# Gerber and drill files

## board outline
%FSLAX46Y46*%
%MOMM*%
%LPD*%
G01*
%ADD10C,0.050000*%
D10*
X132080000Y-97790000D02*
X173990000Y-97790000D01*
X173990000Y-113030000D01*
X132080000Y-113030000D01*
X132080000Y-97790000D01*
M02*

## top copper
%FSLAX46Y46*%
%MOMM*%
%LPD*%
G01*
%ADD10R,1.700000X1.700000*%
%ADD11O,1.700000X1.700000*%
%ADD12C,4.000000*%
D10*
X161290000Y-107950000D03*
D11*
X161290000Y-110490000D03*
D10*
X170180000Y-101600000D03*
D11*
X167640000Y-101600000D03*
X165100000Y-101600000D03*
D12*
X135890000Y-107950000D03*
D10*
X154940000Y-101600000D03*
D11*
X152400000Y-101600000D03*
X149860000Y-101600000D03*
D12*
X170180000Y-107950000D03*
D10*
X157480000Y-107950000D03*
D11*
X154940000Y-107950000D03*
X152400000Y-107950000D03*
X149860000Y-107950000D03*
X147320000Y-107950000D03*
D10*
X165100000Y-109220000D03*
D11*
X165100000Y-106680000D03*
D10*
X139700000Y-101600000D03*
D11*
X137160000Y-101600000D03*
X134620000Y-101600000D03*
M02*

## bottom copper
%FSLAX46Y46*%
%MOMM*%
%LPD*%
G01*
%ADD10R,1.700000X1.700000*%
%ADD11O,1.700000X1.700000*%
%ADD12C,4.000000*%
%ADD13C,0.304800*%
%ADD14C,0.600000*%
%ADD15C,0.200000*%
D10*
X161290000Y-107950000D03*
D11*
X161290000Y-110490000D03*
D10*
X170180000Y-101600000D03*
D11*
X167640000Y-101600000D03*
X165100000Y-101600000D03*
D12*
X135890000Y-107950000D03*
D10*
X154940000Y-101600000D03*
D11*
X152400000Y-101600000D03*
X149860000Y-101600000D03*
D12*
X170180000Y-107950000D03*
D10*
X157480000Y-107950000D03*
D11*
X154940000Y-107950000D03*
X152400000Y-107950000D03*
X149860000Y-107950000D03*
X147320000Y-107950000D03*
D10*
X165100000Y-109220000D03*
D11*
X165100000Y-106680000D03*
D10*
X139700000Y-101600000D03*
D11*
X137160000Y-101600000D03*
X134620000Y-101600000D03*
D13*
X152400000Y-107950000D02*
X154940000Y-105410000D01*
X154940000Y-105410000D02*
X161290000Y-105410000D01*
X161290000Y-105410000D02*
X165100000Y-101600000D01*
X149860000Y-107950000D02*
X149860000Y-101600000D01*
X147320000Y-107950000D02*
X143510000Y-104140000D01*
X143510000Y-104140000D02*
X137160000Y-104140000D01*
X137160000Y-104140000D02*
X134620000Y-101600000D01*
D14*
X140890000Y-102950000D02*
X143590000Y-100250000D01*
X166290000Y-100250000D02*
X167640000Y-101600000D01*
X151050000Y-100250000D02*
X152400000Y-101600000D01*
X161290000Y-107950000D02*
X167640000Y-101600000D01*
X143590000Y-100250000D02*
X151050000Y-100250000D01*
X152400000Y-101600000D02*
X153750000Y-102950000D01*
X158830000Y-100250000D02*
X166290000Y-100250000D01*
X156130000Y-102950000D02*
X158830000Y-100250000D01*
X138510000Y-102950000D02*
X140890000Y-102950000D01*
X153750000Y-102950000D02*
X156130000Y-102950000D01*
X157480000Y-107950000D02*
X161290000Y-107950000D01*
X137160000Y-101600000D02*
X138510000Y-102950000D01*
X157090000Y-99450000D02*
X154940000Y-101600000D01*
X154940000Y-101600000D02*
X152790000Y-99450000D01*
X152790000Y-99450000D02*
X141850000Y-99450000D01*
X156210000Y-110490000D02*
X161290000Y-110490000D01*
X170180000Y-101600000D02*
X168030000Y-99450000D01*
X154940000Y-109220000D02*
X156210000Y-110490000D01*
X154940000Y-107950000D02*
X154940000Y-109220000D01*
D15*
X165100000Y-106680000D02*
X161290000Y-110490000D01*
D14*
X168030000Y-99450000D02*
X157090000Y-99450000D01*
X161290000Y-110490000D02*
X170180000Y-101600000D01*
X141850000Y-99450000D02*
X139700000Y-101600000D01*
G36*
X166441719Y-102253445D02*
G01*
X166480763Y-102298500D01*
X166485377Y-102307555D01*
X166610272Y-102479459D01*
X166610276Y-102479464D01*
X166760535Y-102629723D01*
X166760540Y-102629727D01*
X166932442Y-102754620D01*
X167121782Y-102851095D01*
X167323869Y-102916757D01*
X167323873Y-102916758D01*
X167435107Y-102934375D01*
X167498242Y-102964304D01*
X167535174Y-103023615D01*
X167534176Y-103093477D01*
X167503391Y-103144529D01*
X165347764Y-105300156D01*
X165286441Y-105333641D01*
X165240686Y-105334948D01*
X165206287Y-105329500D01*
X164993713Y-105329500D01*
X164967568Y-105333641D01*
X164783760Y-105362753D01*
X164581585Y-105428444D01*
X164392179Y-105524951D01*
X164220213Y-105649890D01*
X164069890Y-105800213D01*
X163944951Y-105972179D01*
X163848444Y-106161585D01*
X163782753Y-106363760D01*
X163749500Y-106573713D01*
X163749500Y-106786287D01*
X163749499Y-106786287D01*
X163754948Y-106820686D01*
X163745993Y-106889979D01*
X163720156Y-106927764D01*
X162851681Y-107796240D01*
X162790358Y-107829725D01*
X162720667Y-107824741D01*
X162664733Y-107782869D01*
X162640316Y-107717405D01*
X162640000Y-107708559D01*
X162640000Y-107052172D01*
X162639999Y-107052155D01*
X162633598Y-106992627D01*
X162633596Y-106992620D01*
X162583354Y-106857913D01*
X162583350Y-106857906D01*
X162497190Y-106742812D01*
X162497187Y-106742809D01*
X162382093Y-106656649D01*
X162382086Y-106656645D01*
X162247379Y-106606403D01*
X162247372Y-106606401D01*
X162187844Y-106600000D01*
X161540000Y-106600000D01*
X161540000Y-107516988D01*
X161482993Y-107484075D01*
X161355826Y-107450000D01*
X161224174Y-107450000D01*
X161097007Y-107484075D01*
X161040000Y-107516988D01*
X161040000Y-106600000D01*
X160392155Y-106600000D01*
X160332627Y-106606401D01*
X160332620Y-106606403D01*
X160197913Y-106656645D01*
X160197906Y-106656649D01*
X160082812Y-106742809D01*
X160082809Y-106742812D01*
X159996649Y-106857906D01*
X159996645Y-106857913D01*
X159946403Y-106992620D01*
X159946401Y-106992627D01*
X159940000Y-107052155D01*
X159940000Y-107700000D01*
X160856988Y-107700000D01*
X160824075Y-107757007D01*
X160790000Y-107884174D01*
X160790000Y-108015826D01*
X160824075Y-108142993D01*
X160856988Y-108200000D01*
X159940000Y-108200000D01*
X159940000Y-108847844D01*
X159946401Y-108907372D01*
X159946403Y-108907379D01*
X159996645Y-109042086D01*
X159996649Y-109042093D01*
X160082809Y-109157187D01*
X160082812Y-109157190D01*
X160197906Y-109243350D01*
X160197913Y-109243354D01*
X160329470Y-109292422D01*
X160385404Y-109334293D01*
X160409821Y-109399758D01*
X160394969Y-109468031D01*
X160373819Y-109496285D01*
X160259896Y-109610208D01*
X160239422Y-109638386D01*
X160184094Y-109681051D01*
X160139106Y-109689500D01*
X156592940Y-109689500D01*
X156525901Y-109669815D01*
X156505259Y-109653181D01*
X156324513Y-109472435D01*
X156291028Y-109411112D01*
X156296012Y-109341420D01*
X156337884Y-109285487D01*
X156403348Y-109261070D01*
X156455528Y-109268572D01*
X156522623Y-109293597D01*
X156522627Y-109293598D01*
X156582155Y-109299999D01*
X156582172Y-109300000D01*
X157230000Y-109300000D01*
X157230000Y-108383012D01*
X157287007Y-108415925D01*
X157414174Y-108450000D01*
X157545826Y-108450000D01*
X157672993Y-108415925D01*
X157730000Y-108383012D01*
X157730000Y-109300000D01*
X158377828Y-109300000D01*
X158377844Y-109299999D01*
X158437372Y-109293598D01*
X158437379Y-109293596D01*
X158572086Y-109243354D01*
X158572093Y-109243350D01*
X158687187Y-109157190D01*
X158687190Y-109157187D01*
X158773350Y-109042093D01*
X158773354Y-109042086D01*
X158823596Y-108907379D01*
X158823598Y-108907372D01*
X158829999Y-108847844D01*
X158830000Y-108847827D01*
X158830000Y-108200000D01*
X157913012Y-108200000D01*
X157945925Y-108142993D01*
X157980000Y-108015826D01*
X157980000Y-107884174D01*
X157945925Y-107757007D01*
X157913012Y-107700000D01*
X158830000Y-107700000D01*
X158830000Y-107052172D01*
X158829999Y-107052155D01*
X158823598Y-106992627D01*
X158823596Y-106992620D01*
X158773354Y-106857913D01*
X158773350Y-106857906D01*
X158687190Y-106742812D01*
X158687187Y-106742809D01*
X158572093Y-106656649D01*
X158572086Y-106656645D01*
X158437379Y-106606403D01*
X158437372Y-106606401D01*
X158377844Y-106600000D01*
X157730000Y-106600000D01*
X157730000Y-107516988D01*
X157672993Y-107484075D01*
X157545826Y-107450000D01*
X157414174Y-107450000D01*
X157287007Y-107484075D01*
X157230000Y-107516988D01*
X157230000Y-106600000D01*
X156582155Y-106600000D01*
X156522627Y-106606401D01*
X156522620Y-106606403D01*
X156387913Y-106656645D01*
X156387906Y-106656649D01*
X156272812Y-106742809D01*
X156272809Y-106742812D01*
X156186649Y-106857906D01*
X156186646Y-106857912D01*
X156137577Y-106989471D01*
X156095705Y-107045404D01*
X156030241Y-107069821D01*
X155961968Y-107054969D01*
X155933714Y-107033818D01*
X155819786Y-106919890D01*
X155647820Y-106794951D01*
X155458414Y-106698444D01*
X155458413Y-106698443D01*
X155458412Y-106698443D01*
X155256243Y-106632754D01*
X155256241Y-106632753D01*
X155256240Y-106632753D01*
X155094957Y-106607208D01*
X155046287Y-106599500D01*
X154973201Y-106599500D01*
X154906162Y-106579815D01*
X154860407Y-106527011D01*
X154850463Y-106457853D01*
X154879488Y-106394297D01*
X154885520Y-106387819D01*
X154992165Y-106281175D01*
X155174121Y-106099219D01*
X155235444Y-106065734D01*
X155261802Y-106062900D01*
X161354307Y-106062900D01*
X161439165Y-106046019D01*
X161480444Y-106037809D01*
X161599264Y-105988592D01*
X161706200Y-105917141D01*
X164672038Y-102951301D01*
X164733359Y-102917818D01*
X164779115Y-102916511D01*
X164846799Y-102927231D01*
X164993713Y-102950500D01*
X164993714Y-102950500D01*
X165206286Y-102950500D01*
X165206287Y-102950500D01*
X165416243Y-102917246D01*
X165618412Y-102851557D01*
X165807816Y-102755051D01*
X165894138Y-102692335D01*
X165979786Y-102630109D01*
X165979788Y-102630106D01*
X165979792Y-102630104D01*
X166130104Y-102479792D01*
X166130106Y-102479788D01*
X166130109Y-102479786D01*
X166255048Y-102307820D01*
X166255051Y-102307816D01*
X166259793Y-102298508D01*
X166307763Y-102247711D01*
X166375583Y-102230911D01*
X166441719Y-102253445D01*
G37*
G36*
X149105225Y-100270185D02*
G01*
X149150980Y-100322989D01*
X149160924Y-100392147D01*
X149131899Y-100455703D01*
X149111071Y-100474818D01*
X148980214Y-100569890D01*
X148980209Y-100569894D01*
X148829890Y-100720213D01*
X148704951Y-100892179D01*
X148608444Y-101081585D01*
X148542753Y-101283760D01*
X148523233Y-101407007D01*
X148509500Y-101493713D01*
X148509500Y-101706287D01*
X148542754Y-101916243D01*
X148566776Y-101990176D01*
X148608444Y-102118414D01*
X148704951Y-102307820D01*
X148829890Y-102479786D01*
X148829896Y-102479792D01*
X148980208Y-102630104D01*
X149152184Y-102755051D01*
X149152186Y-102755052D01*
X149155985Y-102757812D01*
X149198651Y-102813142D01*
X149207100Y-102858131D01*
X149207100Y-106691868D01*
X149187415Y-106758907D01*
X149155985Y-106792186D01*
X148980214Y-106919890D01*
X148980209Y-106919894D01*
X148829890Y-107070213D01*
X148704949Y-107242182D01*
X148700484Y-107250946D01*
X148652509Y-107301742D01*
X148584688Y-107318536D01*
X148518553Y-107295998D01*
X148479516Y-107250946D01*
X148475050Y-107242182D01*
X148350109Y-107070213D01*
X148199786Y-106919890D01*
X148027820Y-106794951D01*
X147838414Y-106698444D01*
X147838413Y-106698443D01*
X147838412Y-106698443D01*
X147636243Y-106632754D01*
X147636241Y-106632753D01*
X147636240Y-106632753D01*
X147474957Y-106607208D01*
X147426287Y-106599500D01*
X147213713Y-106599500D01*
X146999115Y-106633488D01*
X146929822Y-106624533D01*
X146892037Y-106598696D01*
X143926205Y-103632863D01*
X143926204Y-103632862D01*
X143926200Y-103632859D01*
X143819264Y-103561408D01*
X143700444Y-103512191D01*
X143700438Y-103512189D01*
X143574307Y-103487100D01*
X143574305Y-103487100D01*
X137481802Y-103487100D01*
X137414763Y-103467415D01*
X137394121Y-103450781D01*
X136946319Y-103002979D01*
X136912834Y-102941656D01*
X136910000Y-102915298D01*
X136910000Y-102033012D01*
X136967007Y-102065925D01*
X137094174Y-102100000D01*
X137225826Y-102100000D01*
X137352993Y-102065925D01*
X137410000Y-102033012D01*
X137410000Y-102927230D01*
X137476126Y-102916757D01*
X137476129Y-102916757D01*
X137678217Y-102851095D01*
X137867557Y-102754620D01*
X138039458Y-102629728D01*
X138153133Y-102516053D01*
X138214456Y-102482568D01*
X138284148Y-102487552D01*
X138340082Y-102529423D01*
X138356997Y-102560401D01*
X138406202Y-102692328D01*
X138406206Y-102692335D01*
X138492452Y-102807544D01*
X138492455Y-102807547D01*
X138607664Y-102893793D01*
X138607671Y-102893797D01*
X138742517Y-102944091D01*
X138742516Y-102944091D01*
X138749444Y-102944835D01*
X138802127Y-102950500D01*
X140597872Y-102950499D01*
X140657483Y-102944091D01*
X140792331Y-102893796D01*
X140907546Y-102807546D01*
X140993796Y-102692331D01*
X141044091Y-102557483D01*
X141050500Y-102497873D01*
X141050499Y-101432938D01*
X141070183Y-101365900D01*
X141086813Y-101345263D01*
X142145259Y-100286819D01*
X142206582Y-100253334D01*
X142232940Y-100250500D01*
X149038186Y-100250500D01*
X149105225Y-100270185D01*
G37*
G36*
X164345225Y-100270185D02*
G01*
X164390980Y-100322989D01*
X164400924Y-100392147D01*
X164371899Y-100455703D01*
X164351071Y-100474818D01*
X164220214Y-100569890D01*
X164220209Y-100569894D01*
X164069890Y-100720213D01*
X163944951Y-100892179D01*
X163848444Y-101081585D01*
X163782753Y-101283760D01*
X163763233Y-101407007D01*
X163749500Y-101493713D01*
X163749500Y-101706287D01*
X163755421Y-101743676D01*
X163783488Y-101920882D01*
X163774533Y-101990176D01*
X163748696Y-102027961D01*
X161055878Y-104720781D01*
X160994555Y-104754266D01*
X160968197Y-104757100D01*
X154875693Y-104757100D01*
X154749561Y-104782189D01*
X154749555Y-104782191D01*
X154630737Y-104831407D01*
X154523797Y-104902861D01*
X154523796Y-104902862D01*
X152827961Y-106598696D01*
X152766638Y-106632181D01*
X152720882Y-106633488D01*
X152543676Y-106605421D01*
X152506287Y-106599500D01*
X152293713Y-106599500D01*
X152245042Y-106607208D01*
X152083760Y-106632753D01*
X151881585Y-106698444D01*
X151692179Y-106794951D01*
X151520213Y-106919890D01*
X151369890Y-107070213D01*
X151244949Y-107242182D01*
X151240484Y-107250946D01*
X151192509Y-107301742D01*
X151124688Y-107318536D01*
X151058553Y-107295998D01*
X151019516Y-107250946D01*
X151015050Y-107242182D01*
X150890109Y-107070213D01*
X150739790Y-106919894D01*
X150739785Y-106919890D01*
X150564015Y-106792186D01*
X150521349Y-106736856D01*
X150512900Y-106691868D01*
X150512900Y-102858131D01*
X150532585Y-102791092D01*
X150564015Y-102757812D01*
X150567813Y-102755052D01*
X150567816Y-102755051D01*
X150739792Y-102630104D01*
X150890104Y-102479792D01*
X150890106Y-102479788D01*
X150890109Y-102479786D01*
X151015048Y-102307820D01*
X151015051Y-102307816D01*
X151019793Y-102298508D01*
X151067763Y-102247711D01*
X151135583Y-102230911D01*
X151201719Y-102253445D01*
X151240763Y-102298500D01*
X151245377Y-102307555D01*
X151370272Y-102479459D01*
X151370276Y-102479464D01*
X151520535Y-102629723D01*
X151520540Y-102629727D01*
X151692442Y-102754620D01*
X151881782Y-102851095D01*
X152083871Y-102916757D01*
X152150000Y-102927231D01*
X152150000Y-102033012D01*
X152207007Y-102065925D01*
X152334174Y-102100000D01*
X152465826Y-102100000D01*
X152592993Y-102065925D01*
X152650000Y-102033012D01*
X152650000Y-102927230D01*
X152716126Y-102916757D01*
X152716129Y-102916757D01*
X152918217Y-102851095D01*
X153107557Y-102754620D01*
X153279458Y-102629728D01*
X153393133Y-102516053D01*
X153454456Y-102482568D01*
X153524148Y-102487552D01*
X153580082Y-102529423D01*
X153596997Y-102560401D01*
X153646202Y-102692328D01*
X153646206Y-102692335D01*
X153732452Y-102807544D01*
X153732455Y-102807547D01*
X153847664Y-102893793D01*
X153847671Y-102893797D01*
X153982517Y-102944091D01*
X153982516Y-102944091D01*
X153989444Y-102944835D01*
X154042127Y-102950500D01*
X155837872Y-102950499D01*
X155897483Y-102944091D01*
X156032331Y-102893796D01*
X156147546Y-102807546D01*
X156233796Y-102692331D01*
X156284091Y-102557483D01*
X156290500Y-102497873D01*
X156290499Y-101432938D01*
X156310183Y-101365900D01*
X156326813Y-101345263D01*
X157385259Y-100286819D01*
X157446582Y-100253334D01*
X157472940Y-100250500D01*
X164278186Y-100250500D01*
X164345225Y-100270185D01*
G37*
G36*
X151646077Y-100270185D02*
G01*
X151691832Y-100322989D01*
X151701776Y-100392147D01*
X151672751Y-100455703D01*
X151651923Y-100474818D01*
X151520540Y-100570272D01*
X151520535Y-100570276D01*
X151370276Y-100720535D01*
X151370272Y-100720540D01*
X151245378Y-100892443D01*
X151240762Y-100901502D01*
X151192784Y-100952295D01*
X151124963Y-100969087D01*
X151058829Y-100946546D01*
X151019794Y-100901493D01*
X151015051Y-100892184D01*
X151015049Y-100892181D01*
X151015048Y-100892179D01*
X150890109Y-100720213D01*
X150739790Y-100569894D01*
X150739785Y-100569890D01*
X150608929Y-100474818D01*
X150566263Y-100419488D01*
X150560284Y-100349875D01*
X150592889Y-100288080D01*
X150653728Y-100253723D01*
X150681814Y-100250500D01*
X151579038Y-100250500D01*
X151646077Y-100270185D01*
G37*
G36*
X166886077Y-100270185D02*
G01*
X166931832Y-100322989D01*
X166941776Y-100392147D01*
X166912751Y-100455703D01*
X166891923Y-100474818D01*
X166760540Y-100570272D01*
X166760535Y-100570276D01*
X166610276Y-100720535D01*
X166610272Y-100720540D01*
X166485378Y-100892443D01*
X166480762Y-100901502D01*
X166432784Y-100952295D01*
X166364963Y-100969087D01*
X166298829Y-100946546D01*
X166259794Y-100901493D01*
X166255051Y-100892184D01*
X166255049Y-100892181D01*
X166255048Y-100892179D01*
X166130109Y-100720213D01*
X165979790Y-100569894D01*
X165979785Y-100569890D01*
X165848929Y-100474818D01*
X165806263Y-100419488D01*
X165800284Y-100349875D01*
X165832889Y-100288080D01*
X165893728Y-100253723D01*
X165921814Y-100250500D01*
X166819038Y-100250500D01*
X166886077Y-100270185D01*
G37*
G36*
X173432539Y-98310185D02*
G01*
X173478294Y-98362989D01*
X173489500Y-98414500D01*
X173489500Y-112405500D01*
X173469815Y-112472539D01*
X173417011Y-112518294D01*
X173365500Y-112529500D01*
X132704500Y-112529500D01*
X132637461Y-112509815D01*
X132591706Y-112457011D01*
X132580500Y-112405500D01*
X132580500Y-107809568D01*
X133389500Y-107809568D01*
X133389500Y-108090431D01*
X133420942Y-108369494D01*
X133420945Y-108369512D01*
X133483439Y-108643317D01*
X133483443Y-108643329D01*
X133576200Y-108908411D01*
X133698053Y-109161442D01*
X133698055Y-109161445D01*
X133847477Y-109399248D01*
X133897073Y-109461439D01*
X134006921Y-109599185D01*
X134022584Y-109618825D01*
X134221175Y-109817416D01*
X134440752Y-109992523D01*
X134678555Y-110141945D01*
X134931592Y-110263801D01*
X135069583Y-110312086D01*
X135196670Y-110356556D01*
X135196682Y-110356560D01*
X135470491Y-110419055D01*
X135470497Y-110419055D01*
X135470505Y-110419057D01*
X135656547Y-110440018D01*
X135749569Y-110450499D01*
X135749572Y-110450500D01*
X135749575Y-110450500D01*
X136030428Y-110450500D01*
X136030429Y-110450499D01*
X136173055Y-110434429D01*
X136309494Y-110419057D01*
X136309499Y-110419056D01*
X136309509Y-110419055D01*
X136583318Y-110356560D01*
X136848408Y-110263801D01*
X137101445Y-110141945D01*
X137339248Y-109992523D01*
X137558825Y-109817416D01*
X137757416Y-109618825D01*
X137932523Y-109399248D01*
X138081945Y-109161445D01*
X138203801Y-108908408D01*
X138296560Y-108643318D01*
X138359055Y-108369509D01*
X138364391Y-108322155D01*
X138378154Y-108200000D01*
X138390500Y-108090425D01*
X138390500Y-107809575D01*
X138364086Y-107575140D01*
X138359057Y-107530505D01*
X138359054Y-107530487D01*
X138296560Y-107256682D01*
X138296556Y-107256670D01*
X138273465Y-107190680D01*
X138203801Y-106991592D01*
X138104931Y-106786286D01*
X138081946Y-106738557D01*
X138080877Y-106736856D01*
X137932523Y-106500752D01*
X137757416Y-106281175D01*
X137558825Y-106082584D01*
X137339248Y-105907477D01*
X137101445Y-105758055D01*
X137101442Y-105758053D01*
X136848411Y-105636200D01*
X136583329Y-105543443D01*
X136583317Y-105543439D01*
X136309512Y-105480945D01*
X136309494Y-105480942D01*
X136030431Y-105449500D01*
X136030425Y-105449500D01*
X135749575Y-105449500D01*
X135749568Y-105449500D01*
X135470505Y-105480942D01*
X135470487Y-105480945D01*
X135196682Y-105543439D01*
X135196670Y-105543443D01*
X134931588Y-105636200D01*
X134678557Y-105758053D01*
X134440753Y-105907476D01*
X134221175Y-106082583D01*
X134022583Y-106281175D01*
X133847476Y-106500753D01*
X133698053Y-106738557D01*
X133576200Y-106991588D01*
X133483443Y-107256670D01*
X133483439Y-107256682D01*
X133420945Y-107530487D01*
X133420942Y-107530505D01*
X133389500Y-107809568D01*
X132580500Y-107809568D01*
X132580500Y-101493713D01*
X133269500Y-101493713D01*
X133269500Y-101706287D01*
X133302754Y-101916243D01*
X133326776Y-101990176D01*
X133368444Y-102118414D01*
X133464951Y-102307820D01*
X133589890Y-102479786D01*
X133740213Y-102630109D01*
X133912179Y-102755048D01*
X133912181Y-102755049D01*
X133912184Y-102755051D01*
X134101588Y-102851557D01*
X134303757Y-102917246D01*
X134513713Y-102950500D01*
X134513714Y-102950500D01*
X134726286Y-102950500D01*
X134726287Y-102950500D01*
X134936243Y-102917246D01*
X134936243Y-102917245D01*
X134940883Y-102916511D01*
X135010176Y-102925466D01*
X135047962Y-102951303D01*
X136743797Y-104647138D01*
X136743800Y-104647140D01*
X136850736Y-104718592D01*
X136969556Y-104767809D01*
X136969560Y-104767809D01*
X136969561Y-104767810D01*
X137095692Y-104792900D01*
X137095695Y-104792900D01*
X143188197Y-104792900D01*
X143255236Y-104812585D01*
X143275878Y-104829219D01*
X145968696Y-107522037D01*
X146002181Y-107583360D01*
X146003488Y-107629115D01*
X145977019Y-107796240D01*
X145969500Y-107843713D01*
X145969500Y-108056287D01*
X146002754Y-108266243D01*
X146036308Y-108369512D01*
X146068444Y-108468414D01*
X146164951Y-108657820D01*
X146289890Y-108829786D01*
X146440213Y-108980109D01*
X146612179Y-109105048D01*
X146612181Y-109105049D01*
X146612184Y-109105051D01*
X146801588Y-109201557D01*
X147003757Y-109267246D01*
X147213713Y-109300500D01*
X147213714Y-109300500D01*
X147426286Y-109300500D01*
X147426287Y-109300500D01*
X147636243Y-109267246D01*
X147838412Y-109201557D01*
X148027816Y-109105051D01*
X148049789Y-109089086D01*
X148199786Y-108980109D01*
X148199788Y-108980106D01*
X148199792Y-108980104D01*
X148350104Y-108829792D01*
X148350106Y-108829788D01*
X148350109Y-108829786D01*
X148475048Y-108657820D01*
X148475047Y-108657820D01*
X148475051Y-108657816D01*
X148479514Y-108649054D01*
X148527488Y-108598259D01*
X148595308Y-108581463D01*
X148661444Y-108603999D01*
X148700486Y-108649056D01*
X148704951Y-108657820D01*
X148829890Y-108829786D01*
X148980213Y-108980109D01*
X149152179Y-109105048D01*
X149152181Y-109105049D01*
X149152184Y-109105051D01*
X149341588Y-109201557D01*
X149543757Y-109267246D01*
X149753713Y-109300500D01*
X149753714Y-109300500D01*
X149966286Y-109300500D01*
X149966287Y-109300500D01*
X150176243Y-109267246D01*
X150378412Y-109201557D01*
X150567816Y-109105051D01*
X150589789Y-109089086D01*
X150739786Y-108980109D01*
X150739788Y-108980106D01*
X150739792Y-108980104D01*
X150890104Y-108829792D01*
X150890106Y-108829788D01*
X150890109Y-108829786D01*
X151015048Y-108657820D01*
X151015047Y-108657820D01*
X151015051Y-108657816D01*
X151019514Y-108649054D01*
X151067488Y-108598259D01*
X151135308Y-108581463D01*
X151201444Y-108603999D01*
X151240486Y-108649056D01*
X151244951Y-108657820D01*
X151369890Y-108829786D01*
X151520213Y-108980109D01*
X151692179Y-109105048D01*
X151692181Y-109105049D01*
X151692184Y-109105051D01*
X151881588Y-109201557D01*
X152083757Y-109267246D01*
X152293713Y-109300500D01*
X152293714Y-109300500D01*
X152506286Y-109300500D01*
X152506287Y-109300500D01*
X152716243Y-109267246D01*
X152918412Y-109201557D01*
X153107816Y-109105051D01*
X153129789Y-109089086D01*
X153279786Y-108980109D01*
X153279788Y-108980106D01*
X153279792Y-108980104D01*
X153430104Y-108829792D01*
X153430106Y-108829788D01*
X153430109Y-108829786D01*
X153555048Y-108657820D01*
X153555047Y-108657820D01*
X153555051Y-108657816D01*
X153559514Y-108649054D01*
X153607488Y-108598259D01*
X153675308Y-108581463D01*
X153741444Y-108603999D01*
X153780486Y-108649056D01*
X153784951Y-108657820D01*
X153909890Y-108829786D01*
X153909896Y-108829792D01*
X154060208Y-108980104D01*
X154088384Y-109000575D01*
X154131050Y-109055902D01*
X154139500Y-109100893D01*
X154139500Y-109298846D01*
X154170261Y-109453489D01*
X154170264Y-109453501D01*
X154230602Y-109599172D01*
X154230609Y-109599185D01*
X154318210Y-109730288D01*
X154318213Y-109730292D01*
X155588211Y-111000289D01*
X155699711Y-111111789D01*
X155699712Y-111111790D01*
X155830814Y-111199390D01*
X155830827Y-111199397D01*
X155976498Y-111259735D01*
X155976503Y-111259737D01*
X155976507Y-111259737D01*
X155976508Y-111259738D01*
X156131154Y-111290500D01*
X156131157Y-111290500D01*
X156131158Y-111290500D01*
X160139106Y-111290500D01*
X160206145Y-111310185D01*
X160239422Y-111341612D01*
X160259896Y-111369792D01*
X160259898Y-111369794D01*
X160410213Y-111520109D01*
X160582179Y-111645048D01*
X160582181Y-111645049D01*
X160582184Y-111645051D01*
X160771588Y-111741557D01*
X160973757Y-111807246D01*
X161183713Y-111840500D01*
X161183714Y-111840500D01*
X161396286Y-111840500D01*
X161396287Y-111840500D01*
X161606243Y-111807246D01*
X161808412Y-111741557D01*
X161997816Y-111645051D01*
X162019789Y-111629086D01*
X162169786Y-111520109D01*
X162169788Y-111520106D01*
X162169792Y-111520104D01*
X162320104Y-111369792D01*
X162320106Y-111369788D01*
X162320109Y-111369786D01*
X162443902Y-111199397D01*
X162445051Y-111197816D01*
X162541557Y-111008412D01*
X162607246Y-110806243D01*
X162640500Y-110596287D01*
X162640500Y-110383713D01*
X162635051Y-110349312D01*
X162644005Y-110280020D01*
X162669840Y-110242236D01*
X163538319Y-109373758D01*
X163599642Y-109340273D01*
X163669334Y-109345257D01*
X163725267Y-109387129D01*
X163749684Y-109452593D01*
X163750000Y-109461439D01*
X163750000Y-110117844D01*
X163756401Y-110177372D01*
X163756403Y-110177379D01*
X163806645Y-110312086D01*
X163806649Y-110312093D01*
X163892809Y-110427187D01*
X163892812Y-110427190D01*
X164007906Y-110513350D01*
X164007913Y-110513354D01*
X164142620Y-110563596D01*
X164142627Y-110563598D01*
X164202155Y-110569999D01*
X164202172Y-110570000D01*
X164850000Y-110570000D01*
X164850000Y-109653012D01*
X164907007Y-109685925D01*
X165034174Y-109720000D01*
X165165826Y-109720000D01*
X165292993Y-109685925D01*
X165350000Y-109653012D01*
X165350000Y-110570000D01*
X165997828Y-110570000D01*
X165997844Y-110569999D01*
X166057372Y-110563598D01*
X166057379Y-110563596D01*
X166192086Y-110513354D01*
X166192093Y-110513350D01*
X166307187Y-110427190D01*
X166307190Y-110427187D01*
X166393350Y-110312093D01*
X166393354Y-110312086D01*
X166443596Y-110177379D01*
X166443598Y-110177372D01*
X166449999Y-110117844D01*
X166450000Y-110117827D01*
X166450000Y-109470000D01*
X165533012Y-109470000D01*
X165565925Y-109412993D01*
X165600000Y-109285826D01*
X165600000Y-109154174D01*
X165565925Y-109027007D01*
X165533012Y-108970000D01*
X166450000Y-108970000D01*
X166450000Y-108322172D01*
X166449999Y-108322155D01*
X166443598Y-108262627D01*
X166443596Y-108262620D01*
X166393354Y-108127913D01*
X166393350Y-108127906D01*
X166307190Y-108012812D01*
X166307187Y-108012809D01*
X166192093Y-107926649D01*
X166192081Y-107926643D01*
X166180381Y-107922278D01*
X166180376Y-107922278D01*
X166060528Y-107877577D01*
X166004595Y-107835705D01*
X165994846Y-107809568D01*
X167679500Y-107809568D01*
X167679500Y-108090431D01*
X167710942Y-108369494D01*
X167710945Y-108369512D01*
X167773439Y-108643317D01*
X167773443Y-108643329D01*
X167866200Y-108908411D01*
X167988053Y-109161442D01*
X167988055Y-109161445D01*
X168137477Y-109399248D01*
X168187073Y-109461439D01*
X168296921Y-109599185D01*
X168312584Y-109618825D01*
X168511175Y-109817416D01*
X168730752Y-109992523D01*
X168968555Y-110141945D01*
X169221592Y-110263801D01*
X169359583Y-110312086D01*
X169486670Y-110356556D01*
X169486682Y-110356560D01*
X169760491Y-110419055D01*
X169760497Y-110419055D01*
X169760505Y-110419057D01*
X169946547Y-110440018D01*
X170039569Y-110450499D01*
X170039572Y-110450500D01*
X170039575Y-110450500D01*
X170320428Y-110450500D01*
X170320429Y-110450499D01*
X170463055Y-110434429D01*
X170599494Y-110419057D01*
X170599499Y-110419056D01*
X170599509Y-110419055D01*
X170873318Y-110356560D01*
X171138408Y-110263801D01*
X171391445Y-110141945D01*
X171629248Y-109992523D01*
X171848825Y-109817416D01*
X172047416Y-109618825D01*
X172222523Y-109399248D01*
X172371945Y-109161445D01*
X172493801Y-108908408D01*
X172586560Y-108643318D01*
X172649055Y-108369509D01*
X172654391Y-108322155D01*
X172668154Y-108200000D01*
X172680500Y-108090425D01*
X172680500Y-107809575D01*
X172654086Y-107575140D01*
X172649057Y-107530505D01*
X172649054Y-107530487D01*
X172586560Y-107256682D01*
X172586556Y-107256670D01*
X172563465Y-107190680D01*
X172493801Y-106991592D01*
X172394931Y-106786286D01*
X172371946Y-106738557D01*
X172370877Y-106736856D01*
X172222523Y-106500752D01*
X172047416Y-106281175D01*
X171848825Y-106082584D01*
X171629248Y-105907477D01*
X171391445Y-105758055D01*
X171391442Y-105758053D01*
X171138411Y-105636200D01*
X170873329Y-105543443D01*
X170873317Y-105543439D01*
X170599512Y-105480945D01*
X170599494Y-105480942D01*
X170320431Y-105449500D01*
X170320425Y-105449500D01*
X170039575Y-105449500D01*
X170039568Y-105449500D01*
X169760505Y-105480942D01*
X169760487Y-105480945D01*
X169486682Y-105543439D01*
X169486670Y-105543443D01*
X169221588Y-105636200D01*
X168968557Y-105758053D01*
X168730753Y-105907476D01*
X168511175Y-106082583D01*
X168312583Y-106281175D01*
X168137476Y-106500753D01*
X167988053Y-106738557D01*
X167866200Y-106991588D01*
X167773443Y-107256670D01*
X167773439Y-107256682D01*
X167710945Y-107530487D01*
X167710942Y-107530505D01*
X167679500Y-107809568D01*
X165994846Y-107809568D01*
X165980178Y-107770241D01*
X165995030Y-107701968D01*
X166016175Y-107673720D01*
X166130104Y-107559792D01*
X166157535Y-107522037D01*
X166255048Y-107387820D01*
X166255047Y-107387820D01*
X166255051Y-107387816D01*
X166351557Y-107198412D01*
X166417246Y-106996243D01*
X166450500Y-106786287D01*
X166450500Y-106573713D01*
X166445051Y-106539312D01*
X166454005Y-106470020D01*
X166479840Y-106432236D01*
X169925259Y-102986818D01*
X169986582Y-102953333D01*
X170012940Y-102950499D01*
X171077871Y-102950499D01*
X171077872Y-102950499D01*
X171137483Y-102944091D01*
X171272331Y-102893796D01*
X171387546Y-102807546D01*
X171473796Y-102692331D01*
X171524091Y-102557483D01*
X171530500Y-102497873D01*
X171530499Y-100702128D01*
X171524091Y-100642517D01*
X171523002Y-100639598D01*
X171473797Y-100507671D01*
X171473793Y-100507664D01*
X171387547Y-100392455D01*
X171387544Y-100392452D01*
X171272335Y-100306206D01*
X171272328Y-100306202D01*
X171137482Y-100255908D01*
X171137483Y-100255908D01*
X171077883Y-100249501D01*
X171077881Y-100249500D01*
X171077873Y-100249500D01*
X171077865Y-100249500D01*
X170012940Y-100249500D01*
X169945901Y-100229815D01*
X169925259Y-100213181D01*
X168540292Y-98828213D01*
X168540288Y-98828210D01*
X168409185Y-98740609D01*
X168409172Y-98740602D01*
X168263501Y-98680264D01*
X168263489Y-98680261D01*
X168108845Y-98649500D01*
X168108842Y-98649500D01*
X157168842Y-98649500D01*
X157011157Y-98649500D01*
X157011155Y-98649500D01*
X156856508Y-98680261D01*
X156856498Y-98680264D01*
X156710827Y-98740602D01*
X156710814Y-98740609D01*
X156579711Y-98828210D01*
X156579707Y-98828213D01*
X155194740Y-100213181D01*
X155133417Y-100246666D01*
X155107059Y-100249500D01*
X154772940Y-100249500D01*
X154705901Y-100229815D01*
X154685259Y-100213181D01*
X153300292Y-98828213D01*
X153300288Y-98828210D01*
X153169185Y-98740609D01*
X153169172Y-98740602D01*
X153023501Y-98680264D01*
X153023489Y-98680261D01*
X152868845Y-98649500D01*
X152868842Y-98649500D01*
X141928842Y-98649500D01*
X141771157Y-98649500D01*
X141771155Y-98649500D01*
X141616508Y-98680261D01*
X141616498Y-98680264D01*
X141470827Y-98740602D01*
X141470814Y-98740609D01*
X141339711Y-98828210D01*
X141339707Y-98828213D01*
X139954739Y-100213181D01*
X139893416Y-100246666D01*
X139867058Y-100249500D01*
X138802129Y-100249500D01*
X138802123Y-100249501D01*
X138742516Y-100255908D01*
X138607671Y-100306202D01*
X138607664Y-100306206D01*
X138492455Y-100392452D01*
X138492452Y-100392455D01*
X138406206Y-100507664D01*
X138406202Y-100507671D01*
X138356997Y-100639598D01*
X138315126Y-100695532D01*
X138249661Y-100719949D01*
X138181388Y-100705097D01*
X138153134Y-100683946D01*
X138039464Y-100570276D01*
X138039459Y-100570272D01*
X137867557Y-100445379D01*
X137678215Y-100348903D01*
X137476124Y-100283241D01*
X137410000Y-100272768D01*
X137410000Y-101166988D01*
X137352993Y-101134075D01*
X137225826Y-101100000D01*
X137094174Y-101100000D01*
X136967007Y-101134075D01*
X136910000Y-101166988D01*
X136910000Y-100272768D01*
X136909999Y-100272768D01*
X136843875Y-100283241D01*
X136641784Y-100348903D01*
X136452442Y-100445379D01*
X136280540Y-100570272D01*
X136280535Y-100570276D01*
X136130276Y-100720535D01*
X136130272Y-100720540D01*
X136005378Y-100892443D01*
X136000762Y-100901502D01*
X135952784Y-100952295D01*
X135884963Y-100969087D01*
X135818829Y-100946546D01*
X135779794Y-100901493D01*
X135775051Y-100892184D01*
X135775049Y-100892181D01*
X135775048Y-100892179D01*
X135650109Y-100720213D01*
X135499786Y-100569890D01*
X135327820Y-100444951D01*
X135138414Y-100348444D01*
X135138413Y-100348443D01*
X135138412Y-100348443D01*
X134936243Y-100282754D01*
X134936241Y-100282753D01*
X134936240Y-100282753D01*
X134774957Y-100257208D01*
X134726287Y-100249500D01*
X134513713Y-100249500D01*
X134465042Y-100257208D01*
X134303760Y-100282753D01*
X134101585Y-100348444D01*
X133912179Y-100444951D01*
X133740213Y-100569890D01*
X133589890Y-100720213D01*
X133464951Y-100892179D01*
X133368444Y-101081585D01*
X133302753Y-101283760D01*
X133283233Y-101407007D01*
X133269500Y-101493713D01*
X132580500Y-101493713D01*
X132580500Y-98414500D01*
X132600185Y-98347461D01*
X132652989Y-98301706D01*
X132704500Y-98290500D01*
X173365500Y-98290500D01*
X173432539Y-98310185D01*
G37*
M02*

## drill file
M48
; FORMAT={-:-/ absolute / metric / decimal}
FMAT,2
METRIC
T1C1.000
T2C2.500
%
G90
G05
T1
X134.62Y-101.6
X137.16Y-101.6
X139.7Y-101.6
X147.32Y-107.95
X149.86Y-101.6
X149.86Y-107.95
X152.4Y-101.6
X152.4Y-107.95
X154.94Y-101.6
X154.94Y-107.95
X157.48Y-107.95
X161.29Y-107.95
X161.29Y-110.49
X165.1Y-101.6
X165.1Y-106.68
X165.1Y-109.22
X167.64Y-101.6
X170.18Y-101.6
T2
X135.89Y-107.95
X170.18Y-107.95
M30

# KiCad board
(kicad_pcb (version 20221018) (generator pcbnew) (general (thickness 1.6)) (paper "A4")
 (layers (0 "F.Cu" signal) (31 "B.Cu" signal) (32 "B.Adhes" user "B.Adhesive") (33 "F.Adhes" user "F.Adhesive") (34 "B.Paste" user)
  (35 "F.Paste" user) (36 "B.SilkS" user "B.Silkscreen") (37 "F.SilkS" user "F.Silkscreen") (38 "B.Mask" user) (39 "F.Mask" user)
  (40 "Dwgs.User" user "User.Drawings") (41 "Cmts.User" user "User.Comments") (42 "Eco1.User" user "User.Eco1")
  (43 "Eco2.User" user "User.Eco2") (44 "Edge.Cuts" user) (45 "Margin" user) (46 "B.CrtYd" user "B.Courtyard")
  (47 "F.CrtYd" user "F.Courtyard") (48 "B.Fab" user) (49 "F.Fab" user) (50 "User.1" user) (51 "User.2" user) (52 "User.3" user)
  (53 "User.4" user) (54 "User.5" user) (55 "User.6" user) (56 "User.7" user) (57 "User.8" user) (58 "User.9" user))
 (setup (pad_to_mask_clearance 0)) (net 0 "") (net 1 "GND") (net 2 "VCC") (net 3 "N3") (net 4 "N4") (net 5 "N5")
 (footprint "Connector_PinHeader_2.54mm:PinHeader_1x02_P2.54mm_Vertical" (layer "F.Cu") (at 161.29 107.95)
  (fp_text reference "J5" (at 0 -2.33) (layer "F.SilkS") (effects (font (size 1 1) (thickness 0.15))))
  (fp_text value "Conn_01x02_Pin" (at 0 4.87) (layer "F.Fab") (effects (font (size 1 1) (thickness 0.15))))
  (pad "1" thru_hole rect (at 0 0) (size 1.7 1.7) (drill 1) (layers "*.Cu" "*.Mask") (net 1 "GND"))
  (pad "2" thru_hole oval (at 0 2.54) (size 1.7 1.7) (drill 1) (layers "*.Cu" "*.Mask") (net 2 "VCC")))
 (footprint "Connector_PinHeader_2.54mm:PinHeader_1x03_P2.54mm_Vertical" (layer "F.Cu") (at 170.18 101.6 -90)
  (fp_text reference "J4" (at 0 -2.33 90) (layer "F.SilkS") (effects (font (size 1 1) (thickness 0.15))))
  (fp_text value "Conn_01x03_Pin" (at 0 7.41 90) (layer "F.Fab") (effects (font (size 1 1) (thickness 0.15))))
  (pad "1" thru_hole rect (at 0 0 270) (size 1.7 1.7) (drill 1) (layers "*.Cu" "*.Mask") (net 2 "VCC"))
  (pad "2" thru_hole oval (at 0 2.54 270) (size 1.7 1.7) (drill 1) (layers "*.Cu" "*.Mask") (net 1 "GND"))
  (pad "3" thru_hole oval (at 0 5.08 270) (size 1.7 1.7) (drill 1) (layers "*.Cu" "*.Mask") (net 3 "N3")))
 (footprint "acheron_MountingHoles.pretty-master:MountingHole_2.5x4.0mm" (layer "F.Cu") (at 135.89 107.95)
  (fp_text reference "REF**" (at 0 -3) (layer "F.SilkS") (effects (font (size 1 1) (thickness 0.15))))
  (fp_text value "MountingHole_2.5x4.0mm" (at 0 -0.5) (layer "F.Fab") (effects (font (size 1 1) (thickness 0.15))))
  (pad "1" thru_hole circle (at 0 0) (size 4 4) (drill 2.5) (layers "*.Cu" "*.Mask")))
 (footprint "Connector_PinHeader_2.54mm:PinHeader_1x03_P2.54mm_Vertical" (layer "F.Cu") (at 154.94 101.6 -90)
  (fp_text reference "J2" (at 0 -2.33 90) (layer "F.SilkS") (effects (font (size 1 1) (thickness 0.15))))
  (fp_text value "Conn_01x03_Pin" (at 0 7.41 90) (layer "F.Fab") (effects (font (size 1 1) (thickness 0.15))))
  (pad "1" thru_hole rect (at 0 0 270) (size 1.7 1.7) (drill 1) (layers "*.Cu" "*.Mask") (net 2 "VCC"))
  (pad "2" thru_hole oval (at 0 2.54 270) (size 1.7 1.7) (drill 1) (layers "*.Cu" "*.Mask") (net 1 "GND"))
  (pad "3" thru_hole oval (at 0 5.08 270) (size 1.7 1.7) (drill 1) (layers "*.Cu" "*.Mask") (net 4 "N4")))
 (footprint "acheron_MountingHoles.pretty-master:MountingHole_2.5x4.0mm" (layer "F.Cu") (at 170.18 107.95)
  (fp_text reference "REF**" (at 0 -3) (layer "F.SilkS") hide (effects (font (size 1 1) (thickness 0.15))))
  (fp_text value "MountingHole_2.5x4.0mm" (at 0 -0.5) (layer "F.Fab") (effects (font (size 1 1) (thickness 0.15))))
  (pad "1" thru_hole circle (at 0 0) (size 4 4) (drill 2.5) (layers "*.Cu" "*.Mask")))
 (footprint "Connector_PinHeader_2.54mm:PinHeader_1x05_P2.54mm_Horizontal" (layer "F.Cu") (at 157.48 107.95 -90)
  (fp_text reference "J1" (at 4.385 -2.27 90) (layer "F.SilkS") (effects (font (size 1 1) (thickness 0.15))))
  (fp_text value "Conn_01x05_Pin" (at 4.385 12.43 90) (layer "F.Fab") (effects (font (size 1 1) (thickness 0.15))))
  (pad "1" thru_hole rect (at 0 0 270) (size 1.7 1.7) (drill 1) (layers "*.Cu" "*.Mask") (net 1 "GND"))
  (pad "2" thru_hole oval (at 0 2.54 270) (size 1.7 1.7) (drill 1) (layers "*.Cu" "*.Mask") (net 2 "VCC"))
  (pad "3" thru_hole oval (at 0 5.08 270) (size 1.7 1.7) (drill 1) (layers "*.Cu" "*.Mask") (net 3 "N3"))
  (pad "4" thru_hole oval (at 0 7.62 270) (size 1.7 1.7) (drill 1) (layers "*.Cu" "*.Mask") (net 4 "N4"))
  (pad "5" thru_hole oval (at 0 10.16 270) (size 1.7 1.7) (drill 1) (layers "*.Cu" "*.Mask") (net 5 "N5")))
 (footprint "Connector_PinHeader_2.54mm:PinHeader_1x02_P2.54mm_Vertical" (layer "F.Cu") (at 165.1 109.22 180)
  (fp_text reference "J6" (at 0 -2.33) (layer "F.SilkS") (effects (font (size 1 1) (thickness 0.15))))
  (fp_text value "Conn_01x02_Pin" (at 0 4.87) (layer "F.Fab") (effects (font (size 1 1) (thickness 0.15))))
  (pad "1" thru_hole rect (at 0 0 180) (size 1.7 1.7) (drill 1) (layers "*.Cu" "*.Mask") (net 1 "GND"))
  (pad "2" thru_hole oval (at 0 2.54 180) (size 1.7 1.7) (drill 1) (layers "*.Cu" "*.Mask") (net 2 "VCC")))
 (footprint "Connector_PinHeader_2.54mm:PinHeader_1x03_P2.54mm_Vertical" (layer "F.Cu") (at 139.7 101.6 -90)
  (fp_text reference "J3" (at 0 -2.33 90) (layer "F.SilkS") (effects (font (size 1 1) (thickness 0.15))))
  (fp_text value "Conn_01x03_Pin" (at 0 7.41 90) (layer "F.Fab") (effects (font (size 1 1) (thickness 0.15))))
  (pad "1" thru_hole rect (at 0 0 270) (size 1.7 1.7) (drill 1) (layers "*.Cu" "*.Mask") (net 2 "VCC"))
  (pad "2" thru_hole oval (at 0 2.54 270) (size 1.7 1.7) (drill 1) (layers "*.Cu" "*.Mask") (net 1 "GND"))
  (pad "3" thru_hole oval (at 0 5.08 270) (size 1.7 1.7) (drill 1) (layers "*.Cu" "*.Mask") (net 5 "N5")))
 (gr_rect (start 132.08 97.79) (end 173.99 113.03) (stroke (width 0.05) (type default)) (fill none) (layer "Edge.Cuts"))
 (segment (start 152.4 107.95) (end 154.94 105.41) (width 0.3048) (layer "B.Cu") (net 3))
 (segment (start 154.94 105.41) (end 161.29 105.41) (width 0.3048) (layer "B.Cu") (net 3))
 (segment (start 161.29 105.41) (end 165.1 101.6) (width 0.3048) (layer "B.Cu") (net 3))
 (segment (start 149.86 107.95) (end 149.86 101.6) (width 0.3048) (layer "B.Cu") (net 4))
 (segment (start 147.32 107.95) (end 143.51 104.14) (width 0.3048) (layer "B.Cu") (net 5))
 (segment (start 143.51 104.14) (end 137.16 104.14) (width 0.3048) (layer "B.Cu") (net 5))
 (segment (start 137.16 104.14) (end 134.62 101.6) (width 0.3048) (layer "B.Cu") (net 5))
 (segment (start 140.89 102.95) (end 143.59 100.25) (width 0.6) (layer "B.Cu") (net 1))
 (segment (start 166.29 100.25) (end 167.64 101.6) (width 0.6) (layer "B.Cu") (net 1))
 (segment (start 151.05 100.25) (end 152.4 101.6) (width 0.6) (layer "B.Cu") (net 1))
 (segment (start 161.29 107.95) (end 167.64 101.6) (width 0.6) (layer "B.Cu") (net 1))
 (segment (start 143.59 100.25) (end 151.05 100.25) (width 0.6) (layer "B.Cu") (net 1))
 (segment (start 152.4 101.6) (end 153.75 102.95) (width 0.6) (layer "B.Cu") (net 1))
 (segment (start 158.83 100.25) (end 166.29 100.25) (width 0.6) (layer "B.Cu") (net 1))
 (segment (start 156.13 102.95) (end 158.83 100.25) (width 0.6) (layer "B.Cu") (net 1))
 (segment (start 138.51 102.95) (end 140.89 102.95) (width 0.6) (layer "B.Cu") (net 1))
 (segment (start 153.75 102.95) (end 156.13 102.95) (width 0.6) (layer "B.Cu") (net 1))
 (segment (start 157.48 107.95) (end 161.29 107.95) (width 0.6) (layer "B.Cu") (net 1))
 (segment (start 137.16 101.6) (end 138.51 102.95) (width 0.6) (layer "B.Cu") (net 1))
 (segment (start 157.09 99.45) (end 154.94 101.6) (width 0.6) (layer "B.Cu") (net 2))
 (segment (start 154.94 101.6) (end 152.79 99.45) (width 0.6) (layer "B.Cu") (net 2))
 (segment (start 152.79 99.45) (end 141.85 99.45) (width 0.6) (layer "B.Cu") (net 2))
 (segment (start 156.21 110.49) (end 161.29 110.49) (width 0.6) (layer "B.Cu") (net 2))
 (segment (start 170.18 101.6) (end 168.03 99.45) (width 0.6) (layer "B.Cu") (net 2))
 (segment (start 154.94 109.22) (end 156.21 110.49) (width 0.6) (layer "B.Cu") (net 2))
 (segment (start 154.94 107.95) (end 154.94 109.22) (width 0.6) (layer "B.Cu") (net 2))
 (segment (start 165.1 106.68) (end 161.29 110.49) (width 0.2) (layer "B.Cu") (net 2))
 (segment (start 168.03 99.45) (end 157.09 99.45) (width 0.6) (layer "B.Cu") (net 2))
 (segment (start 161.29 110.49) (end 170.18 101.6) (width 0.6) (layer "B.Cu") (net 2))
 (segment (start 141.85 99.45) (end 139.7 101.6) (width 0.6) (layer "B.Cu") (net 2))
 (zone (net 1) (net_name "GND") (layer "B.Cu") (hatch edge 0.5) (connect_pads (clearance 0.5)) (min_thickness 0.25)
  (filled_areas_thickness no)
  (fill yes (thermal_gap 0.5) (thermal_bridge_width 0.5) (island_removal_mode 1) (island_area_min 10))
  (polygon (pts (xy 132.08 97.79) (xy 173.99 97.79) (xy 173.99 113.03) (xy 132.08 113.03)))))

